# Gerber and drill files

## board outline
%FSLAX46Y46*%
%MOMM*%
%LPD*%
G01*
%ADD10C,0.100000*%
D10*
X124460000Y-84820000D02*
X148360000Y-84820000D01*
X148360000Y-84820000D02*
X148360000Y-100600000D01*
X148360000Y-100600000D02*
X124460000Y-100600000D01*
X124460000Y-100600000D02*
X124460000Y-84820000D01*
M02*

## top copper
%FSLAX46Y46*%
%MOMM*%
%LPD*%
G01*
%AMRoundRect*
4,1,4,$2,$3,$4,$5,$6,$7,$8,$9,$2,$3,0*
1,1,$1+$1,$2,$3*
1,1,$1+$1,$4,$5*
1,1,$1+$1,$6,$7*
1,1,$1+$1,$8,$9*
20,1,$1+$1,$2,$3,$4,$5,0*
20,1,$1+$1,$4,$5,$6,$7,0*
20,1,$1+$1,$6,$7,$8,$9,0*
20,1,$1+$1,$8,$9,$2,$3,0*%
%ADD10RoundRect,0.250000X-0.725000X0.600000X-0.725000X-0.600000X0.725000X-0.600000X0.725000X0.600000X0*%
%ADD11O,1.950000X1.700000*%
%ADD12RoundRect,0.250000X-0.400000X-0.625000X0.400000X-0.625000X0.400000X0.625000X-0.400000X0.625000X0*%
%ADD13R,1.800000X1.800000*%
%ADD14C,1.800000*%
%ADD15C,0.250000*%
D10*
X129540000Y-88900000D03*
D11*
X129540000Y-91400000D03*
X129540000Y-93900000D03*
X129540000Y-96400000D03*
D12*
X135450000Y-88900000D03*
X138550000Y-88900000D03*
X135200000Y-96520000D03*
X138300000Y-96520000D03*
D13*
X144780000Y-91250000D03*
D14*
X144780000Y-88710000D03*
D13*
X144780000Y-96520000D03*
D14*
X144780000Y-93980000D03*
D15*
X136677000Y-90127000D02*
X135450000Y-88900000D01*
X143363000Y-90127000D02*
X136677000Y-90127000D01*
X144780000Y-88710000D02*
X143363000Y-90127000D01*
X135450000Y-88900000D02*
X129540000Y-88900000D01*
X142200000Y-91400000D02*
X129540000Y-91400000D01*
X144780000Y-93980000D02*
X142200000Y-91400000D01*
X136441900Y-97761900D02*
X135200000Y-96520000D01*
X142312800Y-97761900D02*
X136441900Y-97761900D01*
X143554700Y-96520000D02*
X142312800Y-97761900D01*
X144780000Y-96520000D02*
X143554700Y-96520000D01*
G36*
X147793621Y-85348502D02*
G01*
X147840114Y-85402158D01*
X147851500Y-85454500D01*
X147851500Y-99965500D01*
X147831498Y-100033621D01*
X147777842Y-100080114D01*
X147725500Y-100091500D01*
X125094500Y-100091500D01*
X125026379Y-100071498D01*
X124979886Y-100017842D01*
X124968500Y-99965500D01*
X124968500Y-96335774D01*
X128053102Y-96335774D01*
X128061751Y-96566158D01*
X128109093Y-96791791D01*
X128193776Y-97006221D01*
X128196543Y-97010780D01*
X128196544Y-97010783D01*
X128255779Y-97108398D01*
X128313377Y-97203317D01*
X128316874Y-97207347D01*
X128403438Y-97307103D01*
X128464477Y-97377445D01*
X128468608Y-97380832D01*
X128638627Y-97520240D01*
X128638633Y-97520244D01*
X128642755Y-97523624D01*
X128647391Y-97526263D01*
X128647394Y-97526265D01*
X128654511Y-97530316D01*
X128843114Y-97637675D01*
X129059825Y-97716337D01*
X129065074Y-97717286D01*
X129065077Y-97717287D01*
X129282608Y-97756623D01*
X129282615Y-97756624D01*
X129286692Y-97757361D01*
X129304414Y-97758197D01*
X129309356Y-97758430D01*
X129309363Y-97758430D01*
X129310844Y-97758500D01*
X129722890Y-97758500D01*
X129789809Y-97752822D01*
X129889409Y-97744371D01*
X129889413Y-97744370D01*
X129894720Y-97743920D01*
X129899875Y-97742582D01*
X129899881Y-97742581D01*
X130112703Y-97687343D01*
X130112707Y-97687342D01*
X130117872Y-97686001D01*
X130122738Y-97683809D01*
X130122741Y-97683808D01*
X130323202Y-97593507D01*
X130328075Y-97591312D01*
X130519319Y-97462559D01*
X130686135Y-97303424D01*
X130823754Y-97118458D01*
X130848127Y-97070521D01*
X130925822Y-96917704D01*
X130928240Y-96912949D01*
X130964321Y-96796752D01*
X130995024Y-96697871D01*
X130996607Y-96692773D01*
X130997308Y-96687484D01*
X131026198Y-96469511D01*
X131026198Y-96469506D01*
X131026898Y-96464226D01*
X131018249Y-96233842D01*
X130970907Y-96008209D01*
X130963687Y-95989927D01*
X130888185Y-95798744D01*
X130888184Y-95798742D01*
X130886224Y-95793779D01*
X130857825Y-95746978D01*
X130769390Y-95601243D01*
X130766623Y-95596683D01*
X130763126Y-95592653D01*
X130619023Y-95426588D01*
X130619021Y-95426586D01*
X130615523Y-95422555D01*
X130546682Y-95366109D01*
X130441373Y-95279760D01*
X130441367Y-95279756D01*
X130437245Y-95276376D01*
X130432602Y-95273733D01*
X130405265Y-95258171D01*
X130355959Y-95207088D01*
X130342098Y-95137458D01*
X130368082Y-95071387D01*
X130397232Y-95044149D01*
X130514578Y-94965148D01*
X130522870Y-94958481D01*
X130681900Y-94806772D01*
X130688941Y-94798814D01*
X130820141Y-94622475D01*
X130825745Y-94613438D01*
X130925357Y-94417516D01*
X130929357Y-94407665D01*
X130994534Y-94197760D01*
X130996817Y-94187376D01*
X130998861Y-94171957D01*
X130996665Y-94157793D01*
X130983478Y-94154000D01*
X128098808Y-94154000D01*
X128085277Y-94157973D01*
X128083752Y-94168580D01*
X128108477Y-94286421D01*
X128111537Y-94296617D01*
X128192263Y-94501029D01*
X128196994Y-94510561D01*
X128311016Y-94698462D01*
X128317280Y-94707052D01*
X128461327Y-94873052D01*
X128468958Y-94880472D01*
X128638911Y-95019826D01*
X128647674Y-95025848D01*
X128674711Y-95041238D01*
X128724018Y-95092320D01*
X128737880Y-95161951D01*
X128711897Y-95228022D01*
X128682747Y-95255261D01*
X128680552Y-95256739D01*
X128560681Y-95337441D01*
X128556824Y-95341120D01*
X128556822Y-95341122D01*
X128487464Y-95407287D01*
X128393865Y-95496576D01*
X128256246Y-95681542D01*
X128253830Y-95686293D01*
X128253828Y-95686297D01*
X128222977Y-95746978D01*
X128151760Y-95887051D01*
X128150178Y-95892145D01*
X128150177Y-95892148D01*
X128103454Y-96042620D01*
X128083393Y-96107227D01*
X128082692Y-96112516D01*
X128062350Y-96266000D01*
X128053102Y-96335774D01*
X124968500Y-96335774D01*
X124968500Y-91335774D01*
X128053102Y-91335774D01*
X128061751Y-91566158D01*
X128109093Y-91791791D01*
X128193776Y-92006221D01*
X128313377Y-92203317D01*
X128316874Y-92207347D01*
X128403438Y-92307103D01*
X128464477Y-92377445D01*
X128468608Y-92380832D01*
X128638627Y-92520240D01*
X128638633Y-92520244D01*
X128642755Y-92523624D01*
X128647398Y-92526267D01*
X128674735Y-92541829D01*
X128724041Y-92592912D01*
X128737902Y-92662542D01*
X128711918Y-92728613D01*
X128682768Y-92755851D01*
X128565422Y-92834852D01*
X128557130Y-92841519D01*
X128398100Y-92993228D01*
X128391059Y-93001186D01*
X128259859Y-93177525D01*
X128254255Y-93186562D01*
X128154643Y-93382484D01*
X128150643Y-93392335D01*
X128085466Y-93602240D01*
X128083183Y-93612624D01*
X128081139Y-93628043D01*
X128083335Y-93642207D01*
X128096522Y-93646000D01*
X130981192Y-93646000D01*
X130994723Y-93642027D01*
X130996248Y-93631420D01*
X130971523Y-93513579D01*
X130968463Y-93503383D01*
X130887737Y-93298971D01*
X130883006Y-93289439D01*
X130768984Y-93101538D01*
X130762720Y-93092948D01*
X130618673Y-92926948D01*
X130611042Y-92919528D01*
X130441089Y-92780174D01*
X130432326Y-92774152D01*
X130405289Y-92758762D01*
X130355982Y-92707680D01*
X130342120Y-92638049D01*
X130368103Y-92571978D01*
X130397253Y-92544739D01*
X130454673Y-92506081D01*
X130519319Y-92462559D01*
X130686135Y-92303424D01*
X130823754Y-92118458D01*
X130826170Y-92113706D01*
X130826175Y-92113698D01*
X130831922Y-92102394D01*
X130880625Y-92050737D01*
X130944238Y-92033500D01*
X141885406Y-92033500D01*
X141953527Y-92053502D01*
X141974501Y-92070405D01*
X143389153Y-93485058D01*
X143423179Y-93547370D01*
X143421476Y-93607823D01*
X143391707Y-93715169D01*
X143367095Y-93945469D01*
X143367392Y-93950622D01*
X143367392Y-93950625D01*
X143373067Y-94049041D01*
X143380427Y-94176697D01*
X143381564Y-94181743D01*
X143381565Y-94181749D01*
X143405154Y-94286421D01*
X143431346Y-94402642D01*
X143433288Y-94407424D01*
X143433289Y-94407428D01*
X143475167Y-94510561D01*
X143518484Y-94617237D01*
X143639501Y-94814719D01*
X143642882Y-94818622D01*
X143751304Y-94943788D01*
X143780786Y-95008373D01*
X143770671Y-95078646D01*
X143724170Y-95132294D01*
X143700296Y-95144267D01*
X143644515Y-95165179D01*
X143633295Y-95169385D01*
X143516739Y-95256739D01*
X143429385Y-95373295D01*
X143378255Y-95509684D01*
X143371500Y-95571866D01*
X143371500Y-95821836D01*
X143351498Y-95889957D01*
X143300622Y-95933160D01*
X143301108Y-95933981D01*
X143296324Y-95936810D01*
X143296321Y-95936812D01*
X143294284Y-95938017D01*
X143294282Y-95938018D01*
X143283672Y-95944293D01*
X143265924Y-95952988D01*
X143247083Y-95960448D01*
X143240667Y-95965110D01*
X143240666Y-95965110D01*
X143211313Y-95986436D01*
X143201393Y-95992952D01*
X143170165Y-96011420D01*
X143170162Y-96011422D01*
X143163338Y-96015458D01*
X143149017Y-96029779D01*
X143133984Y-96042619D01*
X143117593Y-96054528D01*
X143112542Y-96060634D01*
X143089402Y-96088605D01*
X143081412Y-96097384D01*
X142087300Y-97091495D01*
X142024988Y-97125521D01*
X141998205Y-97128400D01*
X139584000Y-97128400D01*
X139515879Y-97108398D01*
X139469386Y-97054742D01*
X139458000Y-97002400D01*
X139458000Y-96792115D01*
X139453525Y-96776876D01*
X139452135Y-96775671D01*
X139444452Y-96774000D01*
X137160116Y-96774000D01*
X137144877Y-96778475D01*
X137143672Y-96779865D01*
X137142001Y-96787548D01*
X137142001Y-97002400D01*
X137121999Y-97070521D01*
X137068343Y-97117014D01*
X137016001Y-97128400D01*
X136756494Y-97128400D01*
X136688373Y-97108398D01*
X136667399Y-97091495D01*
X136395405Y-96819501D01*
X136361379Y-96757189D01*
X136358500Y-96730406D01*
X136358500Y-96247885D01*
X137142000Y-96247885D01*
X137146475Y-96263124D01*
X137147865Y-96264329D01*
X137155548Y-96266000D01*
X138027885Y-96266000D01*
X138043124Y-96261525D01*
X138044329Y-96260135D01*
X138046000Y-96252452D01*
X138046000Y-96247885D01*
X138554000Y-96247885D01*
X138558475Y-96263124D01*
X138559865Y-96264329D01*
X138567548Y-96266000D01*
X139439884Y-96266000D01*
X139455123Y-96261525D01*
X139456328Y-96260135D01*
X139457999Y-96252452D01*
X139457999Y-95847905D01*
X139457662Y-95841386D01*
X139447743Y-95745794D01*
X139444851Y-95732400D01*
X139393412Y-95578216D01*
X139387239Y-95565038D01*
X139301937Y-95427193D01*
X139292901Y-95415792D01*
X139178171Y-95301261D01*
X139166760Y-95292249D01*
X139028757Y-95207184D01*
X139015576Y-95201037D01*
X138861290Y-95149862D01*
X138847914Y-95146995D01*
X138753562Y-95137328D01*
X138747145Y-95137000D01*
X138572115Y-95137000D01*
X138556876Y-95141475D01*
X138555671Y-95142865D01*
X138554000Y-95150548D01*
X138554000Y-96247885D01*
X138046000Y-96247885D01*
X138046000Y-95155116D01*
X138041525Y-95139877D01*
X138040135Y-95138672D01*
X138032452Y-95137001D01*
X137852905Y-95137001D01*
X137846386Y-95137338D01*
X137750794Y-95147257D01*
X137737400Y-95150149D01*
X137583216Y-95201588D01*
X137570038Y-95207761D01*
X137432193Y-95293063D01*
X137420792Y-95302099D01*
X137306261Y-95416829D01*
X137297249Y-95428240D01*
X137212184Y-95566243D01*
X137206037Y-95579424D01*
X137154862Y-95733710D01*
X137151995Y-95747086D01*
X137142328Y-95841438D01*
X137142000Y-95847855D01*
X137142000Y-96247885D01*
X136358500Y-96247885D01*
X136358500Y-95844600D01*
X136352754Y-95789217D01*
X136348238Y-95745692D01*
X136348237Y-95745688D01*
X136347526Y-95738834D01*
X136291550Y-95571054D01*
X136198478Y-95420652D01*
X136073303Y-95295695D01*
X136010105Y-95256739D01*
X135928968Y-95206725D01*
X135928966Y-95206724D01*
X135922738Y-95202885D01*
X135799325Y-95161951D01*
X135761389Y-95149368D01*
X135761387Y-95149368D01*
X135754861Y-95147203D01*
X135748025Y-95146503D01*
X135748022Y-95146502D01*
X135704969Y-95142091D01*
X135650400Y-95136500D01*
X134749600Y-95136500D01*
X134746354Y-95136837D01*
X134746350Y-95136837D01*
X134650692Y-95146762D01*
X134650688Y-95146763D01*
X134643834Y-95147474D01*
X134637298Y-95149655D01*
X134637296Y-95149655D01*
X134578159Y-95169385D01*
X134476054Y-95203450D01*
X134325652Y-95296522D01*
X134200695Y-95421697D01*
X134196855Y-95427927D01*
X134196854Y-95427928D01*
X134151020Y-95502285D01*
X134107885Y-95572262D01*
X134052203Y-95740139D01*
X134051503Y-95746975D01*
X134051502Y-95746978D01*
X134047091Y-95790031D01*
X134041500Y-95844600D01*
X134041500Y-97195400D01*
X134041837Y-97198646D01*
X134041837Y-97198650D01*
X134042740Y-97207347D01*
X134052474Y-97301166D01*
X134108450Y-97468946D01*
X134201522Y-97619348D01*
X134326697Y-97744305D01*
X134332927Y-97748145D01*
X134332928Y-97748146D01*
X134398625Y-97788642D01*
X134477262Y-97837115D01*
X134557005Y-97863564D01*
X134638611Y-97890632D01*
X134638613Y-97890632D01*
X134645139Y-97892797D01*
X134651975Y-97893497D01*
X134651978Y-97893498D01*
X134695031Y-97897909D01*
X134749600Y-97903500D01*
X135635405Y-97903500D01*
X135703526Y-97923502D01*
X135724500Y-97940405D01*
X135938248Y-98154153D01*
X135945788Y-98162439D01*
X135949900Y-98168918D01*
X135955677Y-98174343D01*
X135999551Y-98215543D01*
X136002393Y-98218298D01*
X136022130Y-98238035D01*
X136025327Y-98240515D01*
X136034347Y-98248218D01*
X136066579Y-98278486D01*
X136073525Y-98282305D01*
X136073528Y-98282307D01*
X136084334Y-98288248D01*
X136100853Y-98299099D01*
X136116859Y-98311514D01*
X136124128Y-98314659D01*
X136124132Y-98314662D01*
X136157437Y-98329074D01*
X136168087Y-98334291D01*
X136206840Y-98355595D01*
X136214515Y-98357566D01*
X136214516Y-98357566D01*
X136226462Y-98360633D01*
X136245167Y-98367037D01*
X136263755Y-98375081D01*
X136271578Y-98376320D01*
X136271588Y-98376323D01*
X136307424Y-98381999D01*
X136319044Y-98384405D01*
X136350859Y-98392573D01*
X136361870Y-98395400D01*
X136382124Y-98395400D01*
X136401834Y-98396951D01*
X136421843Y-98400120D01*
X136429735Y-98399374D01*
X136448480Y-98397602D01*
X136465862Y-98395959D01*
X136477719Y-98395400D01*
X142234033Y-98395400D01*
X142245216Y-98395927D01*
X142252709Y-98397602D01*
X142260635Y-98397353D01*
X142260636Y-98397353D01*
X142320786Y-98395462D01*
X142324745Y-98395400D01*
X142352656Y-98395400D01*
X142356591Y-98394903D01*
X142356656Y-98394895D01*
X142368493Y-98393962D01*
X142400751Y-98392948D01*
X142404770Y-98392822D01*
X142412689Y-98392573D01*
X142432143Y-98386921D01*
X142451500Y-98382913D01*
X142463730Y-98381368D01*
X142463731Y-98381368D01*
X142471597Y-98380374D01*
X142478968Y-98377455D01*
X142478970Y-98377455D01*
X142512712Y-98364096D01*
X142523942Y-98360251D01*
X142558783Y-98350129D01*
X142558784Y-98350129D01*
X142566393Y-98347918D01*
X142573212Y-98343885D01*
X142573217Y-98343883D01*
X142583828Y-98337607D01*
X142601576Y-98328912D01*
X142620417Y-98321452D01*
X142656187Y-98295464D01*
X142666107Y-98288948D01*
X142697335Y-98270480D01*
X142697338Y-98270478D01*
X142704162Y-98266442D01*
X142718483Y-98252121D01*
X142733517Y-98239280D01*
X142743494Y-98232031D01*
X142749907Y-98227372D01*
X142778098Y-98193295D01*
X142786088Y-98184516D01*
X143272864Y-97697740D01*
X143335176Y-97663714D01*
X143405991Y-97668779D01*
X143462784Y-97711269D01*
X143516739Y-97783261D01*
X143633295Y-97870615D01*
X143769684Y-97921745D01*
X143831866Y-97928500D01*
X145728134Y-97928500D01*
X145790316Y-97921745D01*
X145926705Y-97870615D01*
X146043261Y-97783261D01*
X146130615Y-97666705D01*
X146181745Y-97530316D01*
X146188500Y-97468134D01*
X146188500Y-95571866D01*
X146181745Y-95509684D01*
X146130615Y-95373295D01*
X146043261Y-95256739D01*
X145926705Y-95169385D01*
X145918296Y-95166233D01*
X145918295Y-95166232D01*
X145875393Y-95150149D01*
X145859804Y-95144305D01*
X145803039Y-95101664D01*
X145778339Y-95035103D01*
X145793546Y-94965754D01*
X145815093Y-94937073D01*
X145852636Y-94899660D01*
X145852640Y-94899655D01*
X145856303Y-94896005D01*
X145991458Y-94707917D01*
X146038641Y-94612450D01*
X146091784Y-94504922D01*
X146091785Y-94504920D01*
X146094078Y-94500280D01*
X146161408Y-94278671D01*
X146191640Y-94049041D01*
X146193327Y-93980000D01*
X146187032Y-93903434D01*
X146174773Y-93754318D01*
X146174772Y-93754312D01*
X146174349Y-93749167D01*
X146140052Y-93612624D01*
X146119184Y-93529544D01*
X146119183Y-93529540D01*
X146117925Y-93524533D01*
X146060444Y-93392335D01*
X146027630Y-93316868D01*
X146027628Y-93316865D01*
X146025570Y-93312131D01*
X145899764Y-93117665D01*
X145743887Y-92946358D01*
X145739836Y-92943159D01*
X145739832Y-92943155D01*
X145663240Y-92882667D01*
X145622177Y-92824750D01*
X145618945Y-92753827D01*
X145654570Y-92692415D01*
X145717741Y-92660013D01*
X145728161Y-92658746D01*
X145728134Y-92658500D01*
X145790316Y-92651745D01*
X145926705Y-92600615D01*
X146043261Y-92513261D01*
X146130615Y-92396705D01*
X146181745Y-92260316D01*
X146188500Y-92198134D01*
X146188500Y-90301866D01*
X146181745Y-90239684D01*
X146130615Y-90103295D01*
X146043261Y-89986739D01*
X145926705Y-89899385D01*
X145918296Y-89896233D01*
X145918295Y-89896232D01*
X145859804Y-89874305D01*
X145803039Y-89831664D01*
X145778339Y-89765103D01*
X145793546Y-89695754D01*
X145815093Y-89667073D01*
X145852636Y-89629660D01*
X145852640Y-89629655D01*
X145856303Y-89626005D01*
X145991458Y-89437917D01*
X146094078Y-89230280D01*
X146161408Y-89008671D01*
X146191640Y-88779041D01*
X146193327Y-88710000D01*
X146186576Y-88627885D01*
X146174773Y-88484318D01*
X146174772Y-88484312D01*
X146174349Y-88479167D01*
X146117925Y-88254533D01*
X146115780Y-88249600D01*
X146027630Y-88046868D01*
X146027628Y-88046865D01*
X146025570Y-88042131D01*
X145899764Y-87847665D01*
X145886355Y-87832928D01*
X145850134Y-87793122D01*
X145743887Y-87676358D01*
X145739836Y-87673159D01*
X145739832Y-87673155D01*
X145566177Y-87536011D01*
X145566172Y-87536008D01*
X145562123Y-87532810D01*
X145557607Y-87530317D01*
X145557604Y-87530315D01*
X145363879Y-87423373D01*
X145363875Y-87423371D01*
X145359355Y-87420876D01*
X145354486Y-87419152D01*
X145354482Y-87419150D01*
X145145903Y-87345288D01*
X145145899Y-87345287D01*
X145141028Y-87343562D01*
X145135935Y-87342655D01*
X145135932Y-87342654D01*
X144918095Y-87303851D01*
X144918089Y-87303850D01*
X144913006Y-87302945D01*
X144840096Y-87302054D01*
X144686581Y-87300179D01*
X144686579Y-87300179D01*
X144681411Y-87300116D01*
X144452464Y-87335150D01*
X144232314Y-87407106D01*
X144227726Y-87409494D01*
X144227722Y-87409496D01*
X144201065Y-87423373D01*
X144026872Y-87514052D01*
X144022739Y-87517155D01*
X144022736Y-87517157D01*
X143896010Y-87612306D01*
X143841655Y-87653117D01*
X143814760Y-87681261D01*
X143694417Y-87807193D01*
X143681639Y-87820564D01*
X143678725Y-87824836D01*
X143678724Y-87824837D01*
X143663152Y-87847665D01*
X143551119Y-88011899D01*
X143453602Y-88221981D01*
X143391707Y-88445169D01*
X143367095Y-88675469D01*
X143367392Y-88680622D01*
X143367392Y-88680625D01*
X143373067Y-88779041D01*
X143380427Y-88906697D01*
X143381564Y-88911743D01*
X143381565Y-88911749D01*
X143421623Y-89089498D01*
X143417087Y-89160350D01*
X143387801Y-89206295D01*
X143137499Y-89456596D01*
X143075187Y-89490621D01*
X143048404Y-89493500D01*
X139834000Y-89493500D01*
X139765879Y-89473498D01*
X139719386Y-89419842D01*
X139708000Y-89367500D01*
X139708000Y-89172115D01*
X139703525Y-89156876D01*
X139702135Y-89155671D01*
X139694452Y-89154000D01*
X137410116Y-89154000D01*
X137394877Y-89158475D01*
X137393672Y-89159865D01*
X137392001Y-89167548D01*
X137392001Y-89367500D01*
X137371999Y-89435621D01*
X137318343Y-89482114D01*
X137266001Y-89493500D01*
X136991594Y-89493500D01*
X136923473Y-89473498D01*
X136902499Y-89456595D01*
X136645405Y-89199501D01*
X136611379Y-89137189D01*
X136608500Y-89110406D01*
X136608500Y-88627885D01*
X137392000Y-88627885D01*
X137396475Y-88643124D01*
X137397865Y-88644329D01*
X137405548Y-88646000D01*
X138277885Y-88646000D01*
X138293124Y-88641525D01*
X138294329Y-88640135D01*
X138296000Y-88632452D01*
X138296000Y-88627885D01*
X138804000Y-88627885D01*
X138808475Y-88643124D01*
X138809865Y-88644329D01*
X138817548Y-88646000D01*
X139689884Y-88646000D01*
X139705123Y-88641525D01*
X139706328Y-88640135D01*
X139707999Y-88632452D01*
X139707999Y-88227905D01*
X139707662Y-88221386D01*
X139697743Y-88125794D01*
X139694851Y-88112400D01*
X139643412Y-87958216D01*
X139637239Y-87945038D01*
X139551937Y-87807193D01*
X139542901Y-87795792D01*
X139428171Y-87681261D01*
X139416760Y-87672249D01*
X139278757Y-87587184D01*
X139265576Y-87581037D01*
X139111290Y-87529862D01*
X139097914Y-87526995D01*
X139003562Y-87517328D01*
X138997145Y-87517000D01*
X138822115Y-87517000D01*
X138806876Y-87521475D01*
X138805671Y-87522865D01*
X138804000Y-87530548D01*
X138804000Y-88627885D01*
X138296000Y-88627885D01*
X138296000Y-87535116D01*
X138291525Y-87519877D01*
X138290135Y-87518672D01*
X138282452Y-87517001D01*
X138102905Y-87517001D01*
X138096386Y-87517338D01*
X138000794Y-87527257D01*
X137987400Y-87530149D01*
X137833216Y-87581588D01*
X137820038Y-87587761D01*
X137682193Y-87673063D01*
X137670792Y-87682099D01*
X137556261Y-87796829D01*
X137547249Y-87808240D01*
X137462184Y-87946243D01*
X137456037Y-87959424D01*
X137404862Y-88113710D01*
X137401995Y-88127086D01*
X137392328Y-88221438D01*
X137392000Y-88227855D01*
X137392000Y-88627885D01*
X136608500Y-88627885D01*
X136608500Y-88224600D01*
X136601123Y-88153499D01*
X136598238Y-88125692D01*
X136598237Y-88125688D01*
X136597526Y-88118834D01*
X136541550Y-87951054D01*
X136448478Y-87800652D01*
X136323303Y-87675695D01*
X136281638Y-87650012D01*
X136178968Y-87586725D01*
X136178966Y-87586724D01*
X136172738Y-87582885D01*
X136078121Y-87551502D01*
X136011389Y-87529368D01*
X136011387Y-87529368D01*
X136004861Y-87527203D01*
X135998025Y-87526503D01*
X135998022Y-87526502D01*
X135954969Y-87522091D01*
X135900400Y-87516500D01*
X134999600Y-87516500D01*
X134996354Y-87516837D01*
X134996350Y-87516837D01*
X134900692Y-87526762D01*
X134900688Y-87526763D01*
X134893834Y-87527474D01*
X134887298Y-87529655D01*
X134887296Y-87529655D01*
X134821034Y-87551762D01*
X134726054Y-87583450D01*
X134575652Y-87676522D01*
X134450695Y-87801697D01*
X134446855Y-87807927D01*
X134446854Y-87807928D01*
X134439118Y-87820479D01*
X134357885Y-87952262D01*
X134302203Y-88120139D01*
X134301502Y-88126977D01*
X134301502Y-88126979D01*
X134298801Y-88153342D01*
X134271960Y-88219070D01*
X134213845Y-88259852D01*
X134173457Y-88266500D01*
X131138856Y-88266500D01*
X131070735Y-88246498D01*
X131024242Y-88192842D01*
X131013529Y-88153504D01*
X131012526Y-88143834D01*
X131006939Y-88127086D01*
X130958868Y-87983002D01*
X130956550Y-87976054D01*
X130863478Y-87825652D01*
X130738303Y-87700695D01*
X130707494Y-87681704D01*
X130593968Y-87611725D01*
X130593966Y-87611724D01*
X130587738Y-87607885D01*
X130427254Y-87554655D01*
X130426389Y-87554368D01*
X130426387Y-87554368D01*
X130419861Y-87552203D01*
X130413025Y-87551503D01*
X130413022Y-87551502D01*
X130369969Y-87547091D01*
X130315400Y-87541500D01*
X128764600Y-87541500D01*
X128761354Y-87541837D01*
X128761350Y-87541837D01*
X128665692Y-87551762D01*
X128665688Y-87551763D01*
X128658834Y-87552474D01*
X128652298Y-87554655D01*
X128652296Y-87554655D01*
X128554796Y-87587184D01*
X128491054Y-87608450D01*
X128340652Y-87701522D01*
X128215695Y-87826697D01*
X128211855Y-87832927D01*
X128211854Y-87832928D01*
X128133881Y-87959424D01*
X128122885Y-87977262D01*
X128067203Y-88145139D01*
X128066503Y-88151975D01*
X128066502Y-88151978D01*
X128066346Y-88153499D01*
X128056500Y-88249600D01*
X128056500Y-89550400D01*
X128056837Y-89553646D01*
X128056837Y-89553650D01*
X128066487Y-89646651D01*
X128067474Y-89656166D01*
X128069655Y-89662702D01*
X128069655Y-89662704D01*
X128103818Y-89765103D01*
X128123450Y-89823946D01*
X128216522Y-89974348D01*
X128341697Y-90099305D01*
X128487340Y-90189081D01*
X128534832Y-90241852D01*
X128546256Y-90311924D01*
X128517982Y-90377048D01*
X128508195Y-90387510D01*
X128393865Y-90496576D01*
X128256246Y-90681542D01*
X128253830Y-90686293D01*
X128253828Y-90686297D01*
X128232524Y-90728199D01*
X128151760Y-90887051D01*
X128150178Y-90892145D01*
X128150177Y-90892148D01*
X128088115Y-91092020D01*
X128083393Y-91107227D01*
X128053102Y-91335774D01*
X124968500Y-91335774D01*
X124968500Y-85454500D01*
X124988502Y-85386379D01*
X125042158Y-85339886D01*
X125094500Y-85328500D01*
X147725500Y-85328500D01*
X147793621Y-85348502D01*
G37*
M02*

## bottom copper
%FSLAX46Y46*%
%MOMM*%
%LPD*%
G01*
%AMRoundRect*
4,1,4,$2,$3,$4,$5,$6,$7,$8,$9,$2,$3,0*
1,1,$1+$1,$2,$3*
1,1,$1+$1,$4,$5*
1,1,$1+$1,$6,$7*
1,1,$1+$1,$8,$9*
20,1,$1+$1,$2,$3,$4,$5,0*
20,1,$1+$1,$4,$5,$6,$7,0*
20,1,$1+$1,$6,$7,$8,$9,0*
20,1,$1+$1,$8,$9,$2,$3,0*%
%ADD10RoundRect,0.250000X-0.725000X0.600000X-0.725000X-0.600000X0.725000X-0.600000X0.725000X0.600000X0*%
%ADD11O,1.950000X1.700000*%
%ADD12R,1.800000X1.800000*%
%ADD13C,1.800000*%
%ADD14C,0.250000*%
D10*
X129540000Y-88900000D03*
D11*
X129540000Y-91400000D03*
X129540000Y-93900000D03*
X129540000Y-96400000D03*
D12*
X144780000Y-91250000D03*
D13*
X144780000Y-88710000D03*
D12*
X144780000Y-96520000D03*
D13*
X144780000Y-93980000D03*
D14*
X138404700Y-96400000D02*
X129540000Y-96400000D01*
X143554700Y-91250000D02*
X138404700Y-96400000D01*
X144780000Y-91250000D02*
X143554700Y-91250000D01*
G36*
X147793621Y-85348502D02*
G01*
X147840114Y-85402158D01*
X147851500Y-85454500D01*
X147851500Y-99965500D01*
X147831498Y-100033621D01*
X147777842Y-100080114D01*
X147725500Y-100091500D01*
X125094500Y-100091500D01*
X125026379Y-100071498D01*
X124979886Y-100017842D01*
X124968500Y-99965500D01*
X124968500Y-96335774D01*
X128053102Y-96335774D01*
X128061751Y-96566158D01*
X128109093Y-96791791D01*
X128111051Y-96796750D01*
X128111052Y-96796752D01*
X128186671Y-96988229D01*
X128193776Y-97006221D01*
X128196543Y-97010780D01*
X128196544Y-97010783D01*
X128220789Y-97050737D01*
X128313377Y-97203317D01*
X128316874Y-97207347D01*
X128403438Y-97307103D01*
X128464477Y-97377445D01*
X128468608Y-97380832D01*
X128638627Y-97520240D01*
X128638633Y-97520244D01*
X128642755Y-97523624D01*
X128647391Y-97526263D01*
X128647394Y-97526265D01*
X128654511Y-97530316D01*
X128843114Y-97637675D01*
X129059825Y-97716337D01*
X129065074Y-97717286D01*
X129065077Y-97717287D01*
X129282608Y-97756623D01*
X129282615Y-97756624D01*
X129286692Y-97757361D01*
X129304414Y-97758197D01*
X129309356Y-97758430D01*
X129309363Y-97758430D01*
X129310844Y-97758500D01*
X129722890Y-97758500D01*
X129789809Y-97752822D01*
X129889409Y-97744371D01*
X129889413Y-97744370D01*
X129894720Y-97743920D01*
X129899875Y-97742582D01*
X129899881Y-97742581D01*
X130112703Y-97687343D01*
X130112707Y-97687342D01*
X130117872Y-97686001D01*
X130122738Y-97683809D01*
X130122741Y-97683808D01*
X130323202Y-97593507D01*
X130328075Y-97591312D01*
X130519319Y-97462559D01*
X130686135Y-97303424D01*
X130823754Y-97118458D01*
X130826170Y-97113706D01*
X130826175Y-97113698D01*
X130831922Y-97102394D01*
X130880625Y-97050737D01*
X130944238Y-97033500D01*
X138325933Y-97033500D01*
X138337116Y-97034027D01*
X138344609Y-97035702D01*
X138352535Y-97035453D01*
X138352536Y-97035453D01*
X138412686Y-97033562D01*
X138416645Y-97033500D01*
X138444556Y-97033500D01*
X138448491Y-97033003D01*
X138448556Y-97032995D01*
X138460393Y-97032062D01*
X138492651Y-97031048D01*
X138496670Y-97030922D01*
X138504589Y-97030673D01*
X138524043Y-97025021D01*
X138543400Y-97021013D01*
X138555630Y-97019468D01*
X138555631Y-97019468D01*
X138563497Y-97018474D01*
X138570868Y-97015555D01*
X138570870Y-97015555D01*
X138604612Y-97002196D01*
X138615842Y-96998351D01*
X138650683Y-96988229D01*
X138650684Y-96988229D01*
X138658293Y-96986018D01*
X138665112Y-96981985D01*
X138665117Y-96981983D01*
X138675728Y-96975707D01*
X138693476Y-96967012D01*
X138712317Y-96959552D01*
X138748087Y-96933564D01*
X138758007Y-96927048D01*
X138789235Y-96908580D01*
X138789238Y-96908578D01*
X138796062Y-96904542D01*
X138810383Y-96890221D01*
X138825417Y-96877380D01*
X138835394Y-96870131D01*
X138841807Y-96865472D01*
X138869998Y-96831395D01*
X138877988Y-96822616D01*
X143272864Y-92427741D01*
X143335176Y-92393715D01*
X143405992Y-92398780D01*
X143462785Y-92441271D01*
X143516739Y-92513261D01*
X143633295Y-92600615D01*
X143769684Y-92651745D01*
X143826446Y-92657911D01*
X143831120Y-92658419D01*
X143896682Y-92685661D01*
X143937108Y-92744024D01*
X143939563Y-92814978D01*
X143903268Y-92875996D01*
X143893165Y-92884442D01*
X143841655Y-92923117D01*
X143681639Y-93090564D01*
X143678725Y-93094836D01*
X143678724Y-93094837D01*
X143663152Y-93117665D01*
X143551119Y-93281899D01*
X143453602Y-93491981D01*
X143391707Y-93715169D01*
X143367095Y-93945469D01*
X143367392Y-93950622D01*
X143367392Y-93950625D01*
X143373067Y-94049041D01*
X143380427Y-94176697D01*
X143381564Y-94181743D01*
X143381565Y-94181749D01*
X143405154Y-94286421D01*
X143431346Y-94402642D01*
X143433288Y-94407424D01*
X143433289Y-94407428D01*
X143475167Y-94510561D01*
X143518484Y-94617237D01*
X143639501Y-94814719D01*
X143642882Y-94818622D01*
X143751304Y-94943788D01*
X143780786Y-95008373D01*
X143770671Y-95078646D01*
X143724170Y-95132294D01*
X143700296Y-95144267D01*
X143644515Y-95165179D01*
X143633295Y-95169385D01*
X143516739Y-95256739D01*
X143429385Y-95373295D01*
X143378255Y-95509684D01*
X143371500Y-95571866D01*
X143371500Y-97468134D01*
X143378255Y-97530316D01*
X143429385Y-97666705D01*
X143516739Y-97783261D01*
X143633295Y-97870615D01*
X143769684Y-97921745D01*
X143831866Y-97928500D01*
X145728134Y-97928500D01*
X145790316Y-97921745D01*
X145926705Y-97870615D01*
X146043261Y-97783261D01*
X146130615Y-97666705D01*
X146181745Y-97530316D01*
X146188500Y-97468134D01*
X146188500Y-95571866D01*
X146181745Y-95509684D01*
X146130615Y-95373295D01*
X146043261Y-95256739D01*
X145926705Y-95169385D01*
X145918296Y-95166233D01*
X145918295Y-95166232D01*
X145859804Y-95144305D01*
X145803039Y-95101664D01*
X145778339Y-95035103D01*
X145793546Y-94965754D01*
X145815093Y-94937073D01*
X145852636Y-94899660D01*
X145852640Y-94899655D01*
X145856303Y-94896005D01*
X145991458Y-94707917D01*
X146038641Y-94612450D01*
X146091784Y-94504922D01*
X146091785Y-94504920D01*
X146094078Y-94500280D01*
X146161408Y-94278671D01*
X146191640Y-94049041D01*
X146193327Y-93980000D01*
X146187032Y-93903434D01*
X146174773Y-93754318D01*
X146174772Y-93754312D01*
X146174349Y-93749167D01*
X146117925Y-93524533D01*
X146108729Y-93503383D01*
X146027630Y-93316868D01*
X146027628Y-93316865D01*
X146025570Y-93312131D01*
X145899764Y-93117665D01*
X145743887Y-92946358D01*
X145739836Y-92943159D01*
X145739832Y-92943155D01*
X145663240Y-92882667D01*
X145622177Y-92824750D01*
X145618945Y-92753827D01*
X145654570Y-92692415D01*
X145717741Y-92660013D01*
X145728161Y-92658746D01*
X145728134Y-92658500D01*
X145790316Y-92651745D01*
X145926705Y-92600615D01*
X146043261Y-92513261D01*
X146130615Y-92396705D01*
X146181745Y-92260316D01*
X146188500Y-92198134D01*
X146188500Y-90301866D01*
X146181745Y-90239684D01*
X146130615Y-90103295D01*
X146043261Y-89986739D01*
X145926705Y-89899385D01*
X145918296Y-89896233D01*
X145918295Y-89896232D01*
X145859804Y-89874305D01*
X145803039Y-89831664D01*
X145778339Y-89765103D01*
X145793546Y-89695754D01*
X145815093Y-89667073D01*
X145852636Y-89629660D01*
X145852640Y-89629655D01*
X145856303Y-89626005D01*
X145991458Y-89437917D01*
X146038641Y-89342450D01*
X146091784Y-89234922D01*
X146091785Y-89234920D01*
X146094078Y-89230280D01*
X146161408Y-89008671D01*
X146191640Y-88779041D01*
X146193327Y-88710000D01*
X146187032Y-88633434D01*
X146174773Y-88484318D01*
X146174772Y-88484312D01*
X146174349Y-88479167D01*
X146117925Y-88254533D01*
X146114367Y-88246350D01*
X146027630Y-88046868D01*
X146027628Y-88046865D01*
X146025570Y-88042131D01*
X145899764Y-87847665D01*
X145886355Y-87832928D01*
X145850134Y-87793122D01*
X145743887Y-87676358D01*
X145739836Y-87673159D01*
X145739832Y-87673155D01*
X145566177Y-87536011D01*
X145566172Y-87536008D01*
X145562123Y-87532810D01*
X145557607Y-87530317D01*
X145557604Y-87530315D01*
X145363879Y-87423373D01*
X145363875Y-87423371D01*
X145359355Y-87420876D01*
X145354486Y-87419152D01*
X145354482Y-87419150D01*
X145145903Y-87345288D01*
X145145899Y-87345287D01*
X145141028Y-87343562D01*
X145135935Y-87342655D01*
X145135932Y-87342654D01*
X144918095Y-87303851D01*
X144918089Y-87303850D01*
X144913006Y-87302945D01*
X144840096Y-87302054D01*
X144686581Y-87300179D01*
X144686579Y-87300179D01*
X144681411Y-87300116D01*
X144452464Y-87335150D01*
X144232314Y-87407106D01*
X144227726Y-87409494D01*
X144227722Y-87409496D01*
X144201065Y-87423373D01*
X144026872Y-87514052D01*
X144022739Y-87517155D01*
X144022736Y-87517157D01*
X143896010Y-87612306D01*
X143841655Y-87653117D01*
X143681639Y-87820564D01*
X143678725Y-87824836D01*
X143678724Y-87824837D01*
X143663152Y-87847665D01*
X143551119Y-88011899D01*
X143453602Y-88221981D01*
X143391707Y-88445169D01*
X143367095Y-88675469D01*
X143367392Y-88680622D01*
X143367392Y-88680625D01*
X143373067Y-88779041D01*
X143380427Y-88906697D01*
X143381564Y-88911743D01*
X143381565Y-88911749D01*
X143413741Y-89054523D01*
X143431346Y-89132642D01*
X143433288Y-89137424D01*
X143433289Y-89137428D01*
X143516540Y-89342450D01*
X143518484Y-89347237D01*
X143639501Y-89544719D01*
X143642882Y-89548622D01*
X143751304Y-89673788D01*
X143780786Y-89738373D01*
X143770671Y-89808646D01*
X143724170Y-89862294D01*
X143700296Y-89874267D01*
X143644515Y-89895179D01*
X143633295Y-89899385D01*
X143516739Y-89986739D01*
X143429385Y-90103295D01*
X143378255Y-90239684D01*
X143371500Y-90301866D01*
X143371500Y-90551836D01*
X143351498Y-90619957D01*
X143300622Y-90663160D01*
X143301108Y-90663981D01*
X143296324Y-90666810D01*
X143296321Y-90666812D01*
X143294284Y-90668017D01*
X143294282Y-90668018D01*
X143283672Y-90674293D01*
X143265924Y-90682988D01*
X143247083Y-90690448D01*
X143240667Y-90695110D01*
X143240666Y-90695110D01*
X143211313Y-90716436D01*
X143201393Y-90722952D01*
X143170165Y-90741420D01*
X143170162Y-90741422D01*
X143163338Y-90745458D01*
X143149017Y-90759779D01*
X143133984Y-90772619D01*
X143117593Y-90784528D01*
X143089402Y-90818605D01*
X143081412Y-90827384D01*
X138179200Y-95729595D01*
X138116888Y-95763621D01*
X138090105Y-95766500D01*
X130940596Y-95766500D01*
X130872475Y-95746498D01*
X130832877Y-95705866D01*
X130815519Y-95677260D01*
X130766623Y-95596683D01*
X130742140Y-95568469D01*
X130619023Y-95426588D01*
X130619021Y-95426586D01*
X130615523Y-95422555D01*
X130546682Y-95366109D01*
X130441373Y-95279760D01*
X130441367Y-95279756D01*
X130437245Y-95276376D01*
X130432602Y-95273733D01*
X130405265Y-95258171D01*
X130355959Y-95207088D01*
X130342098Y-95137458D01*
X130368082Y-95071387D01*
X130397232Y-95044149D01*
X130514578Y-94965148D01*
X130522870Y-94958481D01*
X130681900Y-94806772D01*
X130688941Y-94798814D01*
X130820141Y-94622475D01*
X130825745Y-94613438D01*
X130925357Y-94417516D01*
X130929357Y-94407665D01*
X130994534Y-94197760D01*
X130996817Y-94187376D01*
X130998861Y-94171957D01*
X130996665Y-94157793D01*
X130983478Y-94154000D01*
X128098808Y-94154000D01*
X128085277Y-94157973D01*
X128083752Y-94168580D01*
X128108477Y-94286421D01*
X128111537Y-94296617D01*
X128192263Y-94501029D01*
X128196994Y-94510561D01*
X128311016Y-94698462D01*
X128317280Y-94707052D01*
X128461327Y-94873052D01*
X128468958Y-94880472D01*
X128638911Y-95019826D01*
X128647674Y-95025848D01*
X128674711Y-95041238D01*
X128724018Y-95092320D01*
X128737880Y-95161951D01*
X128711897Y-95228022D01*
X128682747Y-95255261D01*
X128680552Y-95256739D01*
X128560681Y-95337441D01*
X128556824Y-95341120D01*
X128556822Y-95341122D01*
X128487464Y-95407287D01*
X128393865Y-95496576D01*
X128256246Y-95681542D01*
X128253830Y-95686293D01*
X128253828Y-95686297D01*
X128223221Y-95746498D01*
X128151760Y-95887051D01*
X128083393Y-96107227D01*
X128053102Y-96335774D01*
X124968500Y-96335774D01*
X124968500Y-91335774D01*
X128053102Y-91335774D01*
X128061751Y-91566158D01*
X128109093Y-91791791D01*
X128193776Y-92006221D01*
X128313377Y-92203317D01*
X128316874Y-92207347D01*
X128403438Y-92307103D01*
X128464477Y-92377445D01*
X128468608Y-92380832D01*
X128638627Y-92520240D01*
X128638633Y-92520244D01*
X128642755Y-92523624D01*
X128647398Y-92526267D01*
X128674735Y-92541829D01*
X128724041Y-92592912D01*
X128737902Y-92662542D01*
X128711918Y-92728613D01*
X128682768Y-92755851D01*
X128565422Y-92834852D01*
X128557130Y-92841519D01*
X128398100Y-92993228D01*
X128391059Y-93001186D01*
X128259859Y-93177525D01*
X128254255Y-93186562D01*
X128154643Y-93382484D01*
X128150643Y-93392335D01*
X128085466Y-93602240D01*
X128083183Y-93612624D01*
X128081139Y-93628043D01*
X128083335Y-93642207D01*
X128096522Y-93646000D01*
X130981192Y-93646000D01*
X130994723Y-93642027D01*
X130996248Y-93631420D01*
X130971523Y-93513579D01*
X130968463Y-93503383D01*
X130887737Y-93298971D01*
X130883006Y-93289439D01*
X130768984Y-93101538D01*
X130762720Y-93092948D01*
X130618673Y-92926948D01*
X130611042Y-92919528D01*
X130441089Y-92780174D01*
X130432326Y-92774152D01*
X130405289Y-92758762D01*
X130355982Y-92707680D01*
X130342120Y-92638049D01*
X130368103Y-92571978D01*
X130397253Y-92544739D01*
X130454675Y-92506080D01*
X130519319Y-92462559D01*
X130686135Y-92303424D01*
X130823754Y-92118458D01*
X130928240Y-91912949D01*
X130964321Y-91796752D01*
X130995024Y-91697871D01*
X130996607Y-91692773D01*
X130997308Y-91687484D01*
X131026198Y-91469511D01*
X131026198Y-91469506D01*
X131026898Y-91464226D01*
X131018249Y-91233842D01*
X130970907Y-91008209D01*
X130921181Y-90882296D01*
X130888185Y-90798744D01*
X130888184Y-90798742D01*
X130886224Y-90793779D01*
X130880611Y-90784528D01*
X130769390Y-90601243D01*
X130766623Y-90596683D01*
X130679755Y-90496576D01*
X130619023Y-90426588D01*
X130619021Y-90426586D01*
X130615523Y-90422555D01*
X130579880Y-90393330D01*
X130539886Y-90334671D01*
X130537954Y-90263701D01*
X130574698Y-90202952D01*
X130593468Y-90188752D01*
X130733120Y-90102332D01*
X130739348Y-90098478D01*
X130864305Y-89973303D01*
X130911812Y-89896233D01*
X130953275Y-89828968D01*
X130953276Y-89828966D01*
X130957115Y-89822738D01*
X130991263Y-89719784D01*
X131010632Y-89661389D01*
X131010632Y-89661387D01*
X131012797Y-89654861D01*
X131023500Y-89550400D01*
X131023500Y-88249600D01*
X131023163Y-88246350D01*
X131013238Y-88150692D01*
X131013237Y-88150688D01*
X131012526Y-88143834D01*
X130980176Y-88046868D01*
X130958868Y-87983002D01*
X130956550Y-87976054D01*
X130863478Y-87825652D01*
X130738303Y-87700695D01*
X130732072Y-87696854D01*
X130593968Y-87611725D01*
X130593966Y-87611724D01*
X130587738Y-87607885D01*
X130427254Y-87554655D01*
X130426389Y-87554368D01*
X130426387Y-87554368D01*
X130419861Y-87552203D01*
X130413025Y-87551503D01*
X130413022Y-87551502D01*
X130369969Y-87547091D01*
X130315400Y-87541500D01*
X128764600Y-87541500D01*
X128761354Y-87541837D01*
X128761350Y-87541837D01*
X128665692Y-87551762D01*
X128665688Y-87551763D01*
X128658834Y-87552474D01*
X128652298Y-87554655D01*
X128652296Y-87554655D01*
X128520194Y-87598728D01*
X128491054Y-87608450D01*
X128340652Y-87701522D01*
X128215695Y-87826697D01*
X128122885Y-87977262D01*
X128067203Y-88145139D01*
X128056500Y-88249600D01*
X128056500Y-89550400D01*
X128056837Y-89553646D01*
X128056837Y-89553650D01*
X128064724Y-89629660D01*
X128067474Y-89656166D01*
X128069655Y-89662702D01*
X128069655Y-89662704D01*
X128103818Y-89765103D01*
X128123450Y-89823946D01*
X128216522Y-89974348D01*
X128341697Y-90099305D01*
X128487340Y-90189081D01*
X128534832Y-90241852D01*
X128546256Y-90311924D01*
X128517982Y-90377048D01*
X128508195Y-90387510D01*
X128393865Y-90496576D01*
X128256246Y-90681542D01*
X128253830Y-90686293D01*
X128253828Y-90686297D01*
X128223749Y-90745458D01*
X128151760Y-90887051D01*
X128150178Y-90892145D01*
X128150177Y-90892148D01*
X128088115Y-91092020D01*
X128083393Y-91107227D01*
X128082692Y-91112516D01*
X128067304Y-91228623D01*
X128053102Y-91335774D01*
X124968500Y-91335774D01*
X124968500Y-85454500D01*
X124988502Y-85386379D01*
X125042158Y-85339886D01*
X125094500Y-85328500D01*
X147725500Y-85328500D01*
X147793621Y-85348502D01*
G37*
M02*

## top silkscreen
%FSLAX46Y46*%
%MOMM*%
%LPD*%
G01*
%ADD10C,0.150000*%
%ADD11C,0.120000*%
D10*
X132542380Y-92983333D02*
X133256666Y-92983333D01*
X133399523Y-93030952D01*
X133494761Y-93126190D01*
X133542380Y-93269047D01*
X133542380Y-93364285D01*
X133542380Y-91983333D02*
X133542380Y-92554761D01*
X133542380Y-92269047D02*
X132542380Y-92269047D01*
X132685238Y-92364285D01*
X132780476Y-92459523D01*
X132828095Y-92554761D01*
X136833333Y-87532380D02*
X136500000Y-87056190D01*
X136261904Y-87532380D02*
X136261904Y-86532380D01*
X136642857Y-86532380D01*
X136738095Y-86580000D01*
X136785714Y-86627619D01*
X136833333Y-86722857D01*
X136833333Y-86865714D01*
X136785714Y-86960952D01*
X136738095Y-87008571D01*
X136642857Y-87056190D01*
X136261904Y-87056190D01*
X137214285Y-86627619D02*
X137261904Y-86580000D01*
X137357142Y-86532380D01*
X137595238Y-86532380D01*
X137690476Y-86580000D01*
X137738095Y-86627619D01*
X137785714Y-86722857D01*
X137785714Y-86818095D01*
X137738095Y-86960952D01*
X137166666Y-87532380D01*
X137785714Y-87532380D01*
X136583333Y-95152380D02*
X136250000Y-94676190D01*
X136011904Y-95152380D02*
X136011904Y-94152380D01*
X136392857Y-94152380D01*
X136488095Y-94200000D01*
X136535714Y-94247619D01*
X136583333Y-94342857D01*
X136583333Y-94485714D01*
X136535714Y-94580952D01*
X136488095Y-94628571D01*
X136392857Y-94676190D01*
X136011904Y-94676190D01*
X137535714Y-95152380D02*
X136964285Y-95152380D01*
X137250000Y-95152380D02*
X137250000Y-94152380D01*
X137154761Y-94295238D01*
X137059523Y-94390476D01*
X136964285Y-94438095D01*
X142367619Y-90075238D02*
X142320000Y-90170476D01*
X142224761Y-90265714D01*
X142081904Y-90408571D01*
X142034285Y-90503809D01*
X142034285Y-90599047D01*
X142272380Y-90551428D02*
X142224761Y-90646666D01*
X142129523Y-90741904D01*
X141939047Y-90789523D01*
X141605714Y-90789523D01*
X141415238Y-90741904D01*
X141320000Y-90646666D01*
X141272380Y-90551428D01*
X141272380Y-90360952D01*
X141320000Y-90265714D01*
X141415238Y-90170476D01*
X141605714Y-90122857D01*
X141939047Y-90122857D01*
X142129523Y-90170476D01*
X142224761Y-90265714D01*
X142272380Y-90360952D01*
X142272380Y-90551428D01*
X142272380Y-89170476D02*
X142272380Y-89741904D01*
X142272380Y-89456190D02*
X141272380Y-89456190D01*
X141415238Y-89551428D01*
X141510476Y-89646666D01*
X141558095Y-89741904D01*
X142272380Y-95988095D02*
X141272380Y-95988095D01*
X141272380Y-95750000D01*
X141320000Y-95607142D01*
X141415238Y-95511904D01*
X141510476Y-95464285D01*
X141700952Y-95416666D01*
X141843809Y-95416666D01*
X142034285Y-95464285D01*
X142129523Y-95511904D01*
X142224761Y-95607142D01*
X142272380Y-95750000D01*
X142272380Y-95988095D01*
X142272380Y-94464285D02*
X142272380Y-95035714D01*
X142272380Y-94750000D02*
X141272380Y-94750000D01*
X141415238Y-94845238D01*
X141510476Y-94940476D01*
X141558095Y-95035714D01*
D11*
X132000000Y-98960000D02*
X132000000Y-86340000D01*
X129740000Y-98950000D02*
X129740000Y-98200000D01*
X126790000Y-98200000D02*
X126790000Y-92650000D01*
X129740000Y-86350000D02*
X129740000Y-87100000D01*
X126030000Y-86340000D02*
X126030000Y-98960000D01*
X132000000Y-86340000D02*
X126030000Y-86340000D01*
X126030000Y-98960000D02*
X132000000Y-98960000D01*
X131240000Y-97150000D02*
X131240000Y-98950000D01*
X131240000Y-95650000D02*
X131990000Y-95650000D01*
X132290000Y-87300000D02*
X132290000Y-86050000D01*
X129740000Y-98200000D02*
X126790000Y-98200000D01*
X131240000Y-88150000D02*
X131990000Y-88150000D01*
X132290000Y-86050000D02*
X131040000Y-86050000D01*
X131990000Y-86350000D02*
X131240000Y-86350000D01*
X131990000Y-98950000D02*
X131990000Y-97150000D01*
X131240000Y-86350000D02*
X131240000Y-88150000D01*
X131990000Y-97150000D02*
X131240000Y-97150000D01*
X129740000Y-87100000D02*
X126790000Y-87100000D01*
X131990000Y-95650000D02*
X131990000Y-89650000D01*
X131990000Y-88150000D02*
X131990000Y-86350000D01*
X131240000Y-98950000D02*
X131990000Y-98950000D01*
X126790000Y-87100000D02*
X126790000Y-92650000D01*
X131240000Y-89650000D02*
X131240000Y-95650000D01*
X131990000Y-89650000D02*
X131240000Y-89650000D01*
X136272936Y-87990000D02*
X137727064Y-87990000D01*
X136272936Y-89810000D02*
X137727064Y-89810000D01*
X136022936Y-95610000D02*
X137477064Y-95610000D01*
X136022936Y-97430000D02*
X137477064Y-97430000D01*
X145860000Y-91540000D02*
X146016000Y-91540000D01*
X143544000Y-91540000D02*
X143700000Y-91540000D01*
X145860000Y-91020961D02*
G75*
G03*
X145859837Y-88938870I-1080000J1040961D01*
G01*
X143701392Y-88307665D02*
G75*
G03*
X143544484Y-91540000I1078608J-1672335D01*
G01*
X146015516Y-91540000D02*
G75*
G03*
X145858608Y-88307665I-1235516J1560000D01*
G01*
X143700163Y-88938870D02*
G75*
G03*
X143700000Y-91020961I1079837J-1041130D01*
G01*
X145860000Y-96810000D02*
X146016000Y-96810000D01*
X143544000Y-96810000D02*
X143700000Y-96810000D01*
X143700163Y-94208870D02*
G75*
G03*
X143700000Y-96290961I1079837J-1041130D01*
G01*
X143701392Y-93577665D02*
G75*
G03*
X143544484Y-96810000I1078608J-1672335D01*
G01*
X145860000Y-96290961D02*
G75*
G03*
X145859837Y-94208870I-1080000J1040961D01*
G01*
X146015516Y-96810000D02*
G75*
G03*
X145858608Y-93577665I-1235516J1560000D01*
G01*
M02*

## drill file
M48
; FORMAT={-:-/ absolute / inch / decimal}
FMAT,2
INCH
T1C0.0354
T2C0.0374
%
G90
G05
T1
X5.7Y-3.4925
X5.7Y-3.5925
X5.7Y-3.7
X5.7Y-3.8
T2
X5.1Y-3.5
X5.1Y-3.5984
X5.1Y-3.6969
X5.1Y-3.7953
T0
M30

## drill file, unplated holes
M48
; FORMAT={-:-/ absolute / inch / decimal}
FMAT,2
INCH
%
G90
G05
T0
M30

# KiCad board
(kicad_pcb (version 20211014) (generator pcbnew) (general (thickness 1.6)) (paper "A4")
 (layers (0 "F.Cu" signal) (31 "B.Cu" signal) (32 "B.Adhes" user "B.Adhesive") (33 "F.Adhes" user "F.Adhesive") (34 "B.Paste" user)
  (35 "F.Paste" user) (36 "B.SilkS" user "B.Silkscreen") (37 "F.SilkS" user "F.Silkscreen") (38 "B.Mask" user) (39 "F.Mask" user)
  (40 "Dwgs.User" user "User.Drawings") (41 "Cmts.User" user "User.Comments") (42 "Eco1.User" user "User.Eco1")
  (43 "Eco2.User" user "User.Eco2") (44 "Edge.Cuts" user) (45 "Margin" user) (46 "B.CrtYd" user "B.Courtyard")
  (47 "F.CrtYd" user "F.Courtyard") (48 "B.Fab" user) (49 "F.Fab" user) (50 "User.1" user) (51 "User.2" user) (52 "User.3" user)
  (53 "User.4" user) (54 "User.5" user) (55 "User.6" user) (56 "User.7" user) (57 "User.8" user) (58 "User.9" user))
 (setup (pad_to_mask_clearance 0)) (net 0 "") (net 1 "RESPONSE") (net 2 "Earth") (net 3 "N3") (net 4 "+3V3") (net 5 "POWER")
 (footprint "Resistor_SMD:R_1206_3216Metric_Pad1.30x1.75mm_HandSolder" (layer "F.Cu") (at 137 88.9)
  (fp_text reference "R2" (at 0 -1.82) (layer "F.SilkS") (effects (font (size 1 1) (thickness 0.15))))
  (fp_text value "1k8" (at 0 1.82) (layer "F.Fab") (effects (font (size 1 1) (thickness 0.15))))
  (fp_line (start -0.727064 0.91) (end 0.727064 0.91) (layer "F.SilkS") (width 0.12))
  (fp_line (start -0.727064 -0.91) (end 0.727064 -0.91) (layer "F.SilkS") (width 0.12))
  (pad "1" smd roundrect (at -1.55 0) (size 1.3 1.75) (layers "F.Cu" "F.Paste" "F.Mask") (roundrect_rratio 0.1923076923) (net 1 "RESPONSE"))
  (pad "2" smd roundrect (at 1.55 0) (size 1.3 1.75) (layers "F.Cu" "F.Paste" "F.Mask") (roundrect_rratio 0.1923076923) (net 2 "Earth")))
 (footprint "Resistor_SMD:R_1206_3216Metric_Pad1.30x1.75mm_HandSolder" (layer "F.Cu") (at 136.75 96.52)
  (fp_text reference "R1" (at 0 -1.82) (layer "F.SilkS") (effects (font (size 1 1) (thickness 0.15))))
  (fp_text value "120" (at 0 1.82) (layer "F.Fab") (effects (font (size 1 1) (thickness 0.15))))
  (fp_line (start -0.727064 -0.91) (end 0.727064 -0.91) (layer "F.SilkS") (width 0.12))
  (fp_line (start -0.727064 0.91) (end 0.727064 0.91) (layer "F.SilkS") (width 0.12))
  (pad "1" smd roundrect (at -1.55 0) (size 1.3 1.75) (layers "F.Cu" "F.Paste" "F.Mask") (roundrect_rratio 0.1923076923) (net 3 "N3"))
  (pad "2" smd roundrect (at 1.55 0) (size 1.3 1.75) (layers "F.Cu" "F.Paste" "F.Mask") (roundrect_rratio 0.1923076923) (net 2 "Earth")))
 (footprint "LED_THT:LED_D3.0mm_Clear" (layer "F.Cu") (at 144.78 91.25 90)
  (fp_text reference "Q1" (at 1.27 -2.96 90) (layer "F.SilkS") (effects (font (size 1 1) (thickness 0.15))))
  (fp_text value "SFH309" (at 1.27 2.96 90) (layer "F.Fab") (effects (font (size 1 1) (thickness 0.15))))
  (fp_line (start -0.29 -1.236) (end -0.29 -1.08) (layer "F.SilkS") (width 0.12))
  (fp_line (start -0.29 1.08) (end -0.29 1.236) (layer "F.SilkS") (width 0.12))
  (fp_arc (start 2.942335 1.078608) (mid 1.366487 1.987659) (end -0.29 1.235516) (layer "F.SilkS") (width 0.12))
  (fp_arc (start 2.31113 1.079837) (mid 1.270117 1.5) (end 0.229039 1.08) (layer "F.SilkS") (width 0.12))
  (fp_arc (start -0.29 -1.235516) (mid 1.366487 -1.987659) (end 2.942335 -1.078608) (layer "F.SilkS") (width 0.12))
  (fp_arc (start 0.229039 -1.08) (mid 1.270117 -1.5) (end 2.31113 -1.079837) (layer "F.SilkS") (width 0.12))
  (pad "1" thru_hole rect (at 0 0 90) (size 1.8 1.8) (drill 0.9) (layers *.Cu *.Mask) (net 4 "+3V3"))
  (pad "2" thru_hole circle (at 2.54 0 90) (size 1.8 1.8) (drill 0.9) (layers *.Cu *.Mask) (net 1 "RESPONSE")))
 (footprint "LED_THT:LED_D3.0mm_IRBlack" (layer "F.Cu") (at 144.78 96.52 90)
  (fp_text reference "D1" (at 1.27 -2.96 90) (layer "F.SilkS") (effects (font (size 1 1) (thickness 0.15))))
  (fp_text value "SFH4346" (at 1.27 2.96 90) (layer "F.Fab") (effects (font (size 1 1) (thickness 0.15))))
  (fp_line (start -0.29 1.08) (end -0.29 1.236) (layer "F.SilkS") (width 0.12))
  (fp_line (start -0.29 -1.236) (end -0.29 -1.08) (layer "F.SilkS") (width 0.12))
  (fp_arc (start -0.29 -1.235516) (mid 1.366487 -1.987659) (end 2.942335 -1.078608) (layer "F.SilkS") (width 0.12))
  (fp_arc (start 2.31113 1.079837) (mid 1.270117 1.5) (end 0.229039 1.08) (layer "F.SilkS") (width 0.12))
  (fp_arc (start 2.942335 1.078608) (mid 1.366487 1.987659) (end -0.29 1.235516) (layer "F.SilkS") (width 0.12))
  (fp_arc (start 0.229039 -1.08) (mid 1.270117 -1.5) (end 2.31113 -1.079837) (layer "F.SilkS") (width 0.12))
  (pad "1" thru_hole rect (at 0 0 90) (size 1.8 1.8) (drill 0.9) (layers *.Cu *.Mask) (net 3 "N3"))
  (pad "2" thru_hole circle (at 2.54 0 90) (size 1.8 1.8) (drill 0.9) (layers *.Cu *.Mask) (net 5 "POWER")))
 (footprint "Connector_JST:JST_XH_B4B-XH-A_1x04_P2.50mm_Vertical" (layer "F.Cu") (at 129.54 88.9 -90)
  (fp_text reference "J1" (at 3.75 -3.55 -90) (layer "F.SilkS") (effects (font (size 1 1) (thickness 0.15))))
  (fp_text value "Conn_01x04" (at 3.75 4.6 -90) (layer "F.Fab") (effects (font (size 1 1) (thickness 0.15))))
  (fp_line (start -1.6 -2.75) (end -2.85 -2.75) (layer "F.SilkS") (width 0.12))
  (fp_line (start 0.75 -1.7) (end 6.75 -1.7) (layer "F.SilkS") (width 0.12))
  (fp_line (start 0.75 -2.45) (end 0.75 -1.7) (layer "F.SilkS") (width 0.12))
  (fp_line (start -2.85 -2.75) (end -2.85 -1.5) (layer "F.SilkS") (width 0.12))
  (fp_line (start 8.25 -1.7) (end 10.05 -1.7) (layer "F.SilkS") (width 0.12))
  (fp_line (start -2.55 -1.7) (end -0.75 -1.7) (layer "F.SilkS") (width 0.12))
  (fp_line (start 6.75 -2.45) (end 0.75 -2.45) (layer "F.SilkS") (width 0.12))
  (fp_line (start 10.05 -0.2) (end 9.3 -0.2) (layer "F.SilkS") (width 0.12))
  (fp_line (start 10.05 -1.7) (end 10.05 -2.45) (layer "F.SilkS") (width 0.12))
  (fp_line (start -0.75 -2.45) (end -2.55 -2.45) (layer "F.SilkS") (width 0.12))
  (fp_line (start 10.06 3.51) (end 10.06 -2.46) (layer "F.SilkS") (width 0.12))
  (fp_line (start -1.8 -0.2) (end -1.8 2.75) (layer "F.SilkS") (width 0.12))
  (fp_line (start -2.56 3.51) (end 10.06 3.51) (layer "F.SilkS") (width 0.12))
  (fp_line (start -2.55 -2.45) (end -2.55 -1.7) (layer "F.SilkS") (width 0.12))
  (fp_line (start -2.56 -2.46) (end -2.56 3.51) (layer "F.SilkS") (width 0.12))
  (fp_line (start 6.75 -1.7) (end 6.75 -2.45) (layer "F.SilkS") (width 0.12))
  (fp_line (start -1.8 2.75) (end 3.75 2.75) (layer "F.SilkS") (width 0.12))
  (fp_line (start 10.06 -2.46) (end -2.56 -2.46) (layer "F.SilkS") (width 0.12))
  (fp_line (start -2.55 -0.2) (end -1.8 -0.2) (layer "F.SilkS") (width 0.12))
  (fp_line (start 9.3 -0.2) (end 9.3 2.75) (layer "F.SilkS") (width 0.12))
  (fp_line (start 10.05 -2.45) (end 8.25 -2.45) (layer "F.SilkS") (width 0.12))
  (fp_line (start 9.3 2.75) (end 3.75 2.75) (layer "F.SilkS") (width 0.12))
  (fp_line (start 8.25 -2.45) (end 8.25 -1.7) (layer "F.SilkS") (width 0.12))
  (fp_line (start -0.75 -1.7) (end -0.75 -2.45) (layer "F.SilkS") (width 0.12))
  (pad "1" thru_hole roundrect (at 0 0 270) (size 1.7 1.95) (drill 0.95) (layers *.Cu *.Mask) (roundrect_rratio 0.1470588235)
   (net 1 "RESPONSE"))
  (pad "2" thru_hole oval (at 2.5 0 270) (size 1.7 1.95) (drill 0.95) (layers *.Cu *.Mask) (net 5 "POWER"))
  (pad "3" thru_hole oval (at 5 0 270) (size 1.7 1.95) (drill 0.95) (layers *.Cu *.Mask) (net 2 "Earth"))
  (pad "4" thru_hole oval (at 7.5 0 270) (size 1.7 1.95) (drill 0.95) (layers *.Cu *.Mask) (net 4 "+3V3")))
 (gr_rect (start 124.46 84.82) (end 148.36 100.6) (layer "Edge.Cuts") (width 0.1) (fill none))
 (segment (start 142.3128 97.7619) (end 136.4419 97.7619) (width 0.25) (layer "F.Cu") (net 3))
 (segment (start 136.4419 97.7619) (end 135.2 96.52) (width 0.25) (layer "F.Cu") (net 3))
 (segment (start 144.78 96.52) (end 143.5547 96.52) (width 0.25) (layer "F.Cu") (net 3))
 (segment (start 143.5547 96.52) (end 142.3128 97.7619) (width 0.25) (layer "F.Cu") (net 3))
 (segment (start 144.78 93.98) (end 142.2 91.4) (width 0.25) (layer "F.Cu") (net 5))
 (segment (start 142.2 91.4) (end 129.54 91.4) (width 0.25) (layer "F.Cu") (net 5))
 (segment (start 144.78 88.71) (end 143.363 90.127) (width 0.25) (layer "F.Cu") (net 1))
 (segment (start 136.677 90.127) (end 135.45 88.9) (width 0.25) (layer "F.Cu") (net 1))
 (segment (start 135.45 88.9) (end 129.54 88.9) (width 0.25) (layer "F.Cu") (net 1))
 (segment (start 143.363 90.127) (end 136.677 90.127) (width 0.25) (layer "F.Cu") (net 1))
 (segment (start 144.78 91.25) (end 143.5547 91.25) (width 0.25) (layer "B.Cu") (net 4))
 (segment (start 138.4047 96.4) (end 129.54 96.4) (width 0.25) (layer "B.Cu") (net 4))
 (segment (start 143.5547 91.25) (end 138.4047 96.4) (width 0.25) (layer "B.Cu") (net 4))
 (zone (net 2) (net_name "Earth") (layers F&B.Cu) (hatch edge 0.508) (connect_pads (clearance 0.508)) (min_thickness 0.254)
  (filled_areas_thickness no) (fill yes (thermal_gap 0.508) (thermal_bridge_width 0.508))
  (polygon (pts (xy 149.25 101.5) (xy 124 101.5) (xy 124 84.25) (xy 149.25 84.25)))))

